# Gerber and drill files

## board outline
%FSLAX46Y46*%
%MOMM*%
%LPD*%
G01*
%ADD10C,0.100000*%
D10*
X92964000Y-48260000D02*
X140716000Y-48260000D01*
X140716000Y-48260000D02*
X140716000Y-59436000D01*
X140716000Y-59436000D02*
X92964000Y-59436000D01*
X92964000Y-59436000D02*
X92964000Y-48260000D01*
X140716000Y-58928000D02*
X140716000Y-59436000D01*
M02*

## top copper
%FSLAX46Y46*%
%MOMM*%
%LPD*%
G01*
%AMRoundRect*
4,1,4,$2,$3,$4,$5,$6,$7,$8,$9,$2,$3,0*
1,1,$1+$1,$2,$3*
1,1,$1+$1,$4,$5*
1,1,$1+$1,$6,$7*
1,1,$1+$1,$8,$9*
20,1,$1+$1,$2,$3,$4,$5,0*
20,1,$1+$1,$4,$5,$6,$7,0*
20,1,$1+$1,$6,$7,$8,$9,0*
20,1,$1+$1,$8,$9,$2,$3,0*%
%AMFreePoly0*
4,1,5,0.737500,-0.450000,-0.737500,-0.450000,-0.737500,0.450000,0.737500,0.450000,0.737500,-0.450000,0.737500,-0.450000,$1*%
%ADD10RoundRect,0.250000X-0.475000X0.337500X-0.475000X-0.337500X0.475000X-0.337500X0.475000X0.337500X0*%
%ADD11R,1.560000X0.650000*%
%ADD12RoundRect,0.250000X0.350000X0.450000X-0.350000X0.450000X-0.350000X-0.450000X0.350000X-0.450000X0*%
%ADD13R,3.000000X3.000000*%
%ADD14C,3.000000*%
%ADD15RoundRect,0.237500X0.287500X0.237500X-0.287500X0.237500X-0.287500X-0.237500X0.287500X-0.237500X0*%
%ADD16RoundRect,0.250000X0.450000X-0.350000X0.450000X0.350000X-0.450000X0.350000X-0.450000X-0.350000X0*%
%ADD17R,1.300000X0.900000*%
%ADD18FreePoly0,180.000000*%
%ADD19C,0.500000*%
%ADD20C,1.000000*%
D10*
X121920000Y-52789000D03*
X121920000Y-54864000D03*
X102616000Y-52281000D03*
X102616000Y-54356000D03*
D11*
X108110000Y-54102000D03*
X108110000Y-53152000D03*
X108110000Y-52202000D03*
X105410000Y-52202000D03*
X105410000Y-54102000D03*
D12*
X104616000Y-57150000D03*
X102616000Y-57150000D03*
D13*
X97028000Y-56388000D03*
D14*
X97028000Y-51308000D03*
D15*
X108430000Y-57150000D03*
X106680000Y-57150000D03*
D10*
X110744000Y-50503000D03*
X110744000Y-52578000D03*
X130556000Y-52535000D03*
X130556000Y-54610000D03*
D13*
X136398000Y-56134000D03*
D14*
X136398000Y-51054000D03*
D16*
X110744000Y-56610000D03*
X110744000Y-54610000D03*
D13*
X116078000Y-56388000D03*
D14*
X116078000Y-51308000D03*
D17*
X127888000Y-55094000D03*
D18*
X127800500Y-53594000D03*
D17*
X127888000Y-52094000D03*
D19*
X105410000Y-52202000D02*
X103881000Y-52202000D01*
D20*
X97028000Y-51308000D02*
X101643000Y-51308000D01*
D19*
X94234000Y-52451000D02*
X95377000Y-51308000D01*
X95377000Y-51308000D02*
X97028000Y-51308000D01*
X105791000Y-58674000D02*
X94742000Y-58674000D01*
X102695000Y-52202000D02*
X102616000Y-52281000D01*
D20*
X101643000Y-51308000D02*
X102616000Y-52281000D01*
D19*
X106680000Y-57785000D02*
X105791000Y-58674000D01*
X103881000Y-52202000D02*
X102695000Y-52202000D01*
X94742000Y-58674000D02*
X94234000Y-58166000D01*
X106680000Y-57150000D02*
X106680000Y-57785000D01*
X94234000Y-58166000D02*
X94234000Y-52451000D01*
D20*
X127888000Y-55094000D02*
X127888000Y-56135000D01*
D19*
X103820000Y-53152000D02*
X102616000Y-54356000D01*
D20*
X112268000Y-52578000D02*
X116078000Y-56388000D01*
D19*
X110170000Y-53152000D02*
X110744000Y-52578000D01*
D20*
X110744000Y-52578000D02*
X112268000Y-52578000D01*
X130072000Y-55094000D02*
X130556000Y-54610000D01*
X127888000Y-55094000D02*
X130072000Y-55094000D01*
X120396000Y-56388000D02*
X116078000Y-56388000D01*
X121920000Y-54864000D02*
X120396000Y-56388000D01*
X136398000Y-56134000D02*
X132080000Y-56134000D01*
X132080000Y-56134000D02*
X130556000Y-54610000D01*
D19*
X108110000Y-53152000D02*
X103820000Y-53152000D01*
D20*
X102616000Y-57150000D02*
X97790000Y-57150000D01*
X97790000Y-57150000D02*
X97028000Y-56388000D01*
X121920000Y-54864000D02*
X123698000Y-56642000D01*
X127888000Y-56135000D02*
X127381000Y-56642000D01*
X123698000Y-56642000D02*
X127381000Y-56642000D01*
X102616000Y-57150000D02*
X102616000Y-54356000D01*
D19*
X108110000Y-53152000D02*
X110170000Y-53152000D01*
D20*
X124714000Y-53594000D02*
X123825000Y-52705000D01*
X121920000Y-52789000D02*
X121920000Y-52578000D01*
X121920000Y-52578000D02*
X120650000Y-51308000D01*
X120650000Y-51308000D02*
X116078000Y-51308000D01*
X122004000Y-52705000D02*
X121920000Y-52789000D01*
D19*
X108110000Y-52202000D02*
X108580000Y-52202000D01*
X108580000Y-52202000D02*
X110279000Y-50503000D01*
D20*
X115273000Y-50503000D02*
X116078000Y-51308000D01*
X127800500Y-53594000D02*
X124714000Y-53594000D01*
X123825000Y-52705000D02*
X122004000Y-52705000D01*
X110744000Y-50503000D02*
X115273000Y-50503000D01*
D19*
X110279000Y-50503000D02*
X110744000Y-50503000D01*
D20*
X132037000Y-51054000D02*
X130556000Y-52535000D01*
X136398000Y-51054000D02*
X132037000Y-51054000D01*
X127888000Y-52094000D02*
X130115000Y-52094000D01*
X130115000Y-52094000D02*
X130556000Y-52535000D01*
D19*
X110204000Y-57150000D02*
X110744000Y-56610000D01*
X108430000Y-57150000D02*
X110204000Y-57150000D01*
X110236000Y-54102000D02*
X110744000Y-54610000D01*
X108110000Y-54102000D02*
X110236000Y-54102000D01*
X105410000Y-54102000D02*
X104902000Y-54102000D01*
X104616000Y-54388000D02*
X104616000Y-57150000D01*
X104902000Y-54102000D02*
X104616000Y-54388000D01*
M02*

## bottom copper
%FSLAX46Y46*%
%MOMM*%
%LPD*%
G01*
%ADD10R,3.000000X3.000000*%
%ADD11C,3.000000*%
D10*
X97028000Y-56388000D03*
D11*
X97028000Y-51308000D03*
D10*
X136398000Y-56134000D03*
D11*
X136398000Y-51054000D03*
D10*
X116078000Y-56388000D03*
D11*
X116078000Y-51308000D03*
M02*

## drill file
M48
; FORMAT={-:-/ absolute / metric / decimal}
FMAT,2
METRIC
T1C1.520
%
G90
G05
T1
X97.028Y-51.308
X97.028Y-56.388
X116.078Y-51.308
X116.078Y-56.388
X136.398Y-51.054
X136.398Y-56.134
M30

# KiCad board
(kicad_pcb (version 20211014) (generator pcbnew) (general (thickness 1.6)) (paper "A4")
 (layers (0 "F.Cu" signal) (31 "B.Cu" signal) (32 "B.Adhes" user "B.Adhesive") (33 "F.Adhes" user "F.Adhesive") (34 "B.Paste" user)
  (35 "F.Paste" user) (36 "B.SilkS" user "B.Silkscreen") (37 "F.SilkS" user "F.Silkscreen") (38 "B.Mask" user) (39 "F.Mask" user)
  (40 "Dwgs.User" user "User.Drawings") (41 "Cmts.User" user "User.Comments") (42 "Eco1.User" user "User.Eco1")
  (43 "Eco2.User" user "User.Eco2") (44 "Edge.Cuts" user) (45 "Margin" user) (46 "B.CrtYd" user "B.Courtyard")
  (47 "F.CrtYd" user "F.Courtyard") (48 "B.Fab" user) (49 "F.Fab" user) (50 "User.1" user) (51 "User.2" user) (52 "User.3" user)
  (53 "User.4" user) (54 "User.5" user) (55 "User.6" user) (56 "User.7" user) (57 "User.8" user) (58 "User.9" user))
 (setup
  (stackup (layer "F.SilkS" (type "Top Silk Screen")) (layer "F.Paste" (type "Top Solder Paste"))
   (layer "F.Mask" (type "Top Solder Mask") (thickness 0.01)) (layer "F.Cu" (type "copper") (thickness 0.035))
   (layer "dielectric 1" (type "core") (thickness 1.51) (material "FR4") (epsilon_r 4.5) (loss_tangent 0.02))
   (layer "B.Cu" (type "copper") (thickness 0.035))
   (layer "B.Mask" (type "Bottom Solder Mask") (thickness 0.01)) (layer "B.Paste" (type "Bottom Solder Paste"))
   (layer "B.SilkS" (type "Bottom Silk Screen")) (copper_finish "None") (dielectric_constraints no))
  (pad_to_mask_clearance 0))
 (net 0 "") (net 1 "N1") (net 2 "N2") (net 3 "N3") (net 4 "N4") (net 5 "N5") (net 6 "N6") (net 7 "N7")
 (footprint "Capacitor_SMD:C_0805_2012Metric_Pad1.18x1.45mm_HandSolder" (layer "F.Cu") (at 121.92 53.8265 -90)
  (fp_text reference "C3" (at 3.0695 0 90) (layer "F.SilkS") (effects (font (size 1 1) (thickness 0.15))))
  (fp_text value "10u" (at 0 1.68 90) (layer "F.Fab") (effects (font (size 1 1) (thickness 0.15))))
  (pad "1" smd roundrect (at -1.0375 0 270) (size 1.175 1.45) (layers "F.Cu" "F.Paste" "F.Mask") (roundrect_rratio 0.212766) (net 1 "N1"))
  (pad "2" smd roundrect (at 1.0375 0 270) (size 1.175 1.45) (layers "F.Cu" "F.Paste" "F.Mask") (roundrect_rratio 0.212766) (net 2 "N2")))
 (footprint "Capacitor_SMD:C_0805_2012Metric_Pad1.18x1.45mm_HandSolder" (layer "F.Cu") (at 102.616 53.3185 -90)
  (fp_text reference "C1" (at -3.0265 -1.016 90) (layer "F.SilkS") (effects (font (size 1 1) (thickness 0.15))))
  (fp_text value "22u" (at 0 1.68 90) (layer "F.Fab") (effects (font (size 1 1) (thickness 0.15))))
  (pad "1" smd roundrect (at -1.0375 0 270) (size 1.175 1.45) (layers "F.Cu" "F.Paste" "F.Mask") (roundrect_rratio 0.212766) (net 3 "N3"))
  (pad "2" smd roundrect (at 1.0375 0 270) (size 1.175 1.45) (layers "F.Cu" "F.Paste" "F.Mask") (roundrect_rratio 0.212766) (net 2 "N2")))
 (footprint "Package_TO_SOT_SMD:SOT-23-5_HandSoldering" (layer "F.Cu") (at 106.76 53.152 180)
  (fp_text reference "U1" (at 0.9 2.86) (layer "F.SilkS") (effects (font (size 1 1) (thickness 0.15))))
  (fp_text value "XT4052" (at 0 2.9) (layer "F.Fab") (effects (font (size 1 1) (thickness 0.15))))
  (pad "1" smd rect (at -1.35 -0.95 180) (size 1.56 0.65) (layers "F.Cu" "F.Paste" "F.Mask") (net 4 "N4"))
  (pad "2" smd rect (at -1.35 0 180) (size 1.56 0.65) (layers "F.Cu" "F.Paste" "F.Mask") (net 2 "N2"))
  (pad "3" smd rect (at -1.35 0.95 180) (size 1.56 0.65) (layers "F.Cu" "F.Paste" "F.Mask") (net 1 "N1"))
  (pad "4" smd rect (at 1.35 0.95 180) (size 1.56 0.65) (layers "F.Cu" "F.Paste" "F.Mask") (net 3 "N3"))
  (pad "5" smd rect (at 1.35 -0.95 180) (size 1.56 0.65) (layers "F.Cu" "F.Paste" "F.Mask") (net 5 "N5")))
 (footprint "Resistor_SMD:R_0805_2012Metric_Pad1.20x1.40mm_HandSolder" (layer "F.Cu") (at 103.616 57.15 180)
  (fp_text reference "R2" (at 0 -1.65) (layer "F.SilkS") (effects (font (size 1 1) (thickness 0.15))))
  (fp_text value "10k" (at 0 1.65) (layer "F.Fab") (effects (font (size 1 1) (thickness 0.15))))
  (pad "1" smd roundrect (at -1 0 180) (size 1.2 1.4) (layers "F.Cu" "F.Paste" "F.Mask") (roundrect_rratio 0.208333) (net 5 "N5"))
  (pad "2" smd roundrect (at 1 0 180) (size 1.2 1.4) (layers "F.Cu" "F.Paste" "F.Mask") (roundrect_rratio 0.208333) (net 2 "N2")))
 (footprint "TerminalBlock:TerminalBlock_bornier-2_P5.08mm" (layer "F.Cu") (at 97.028 56.388 90)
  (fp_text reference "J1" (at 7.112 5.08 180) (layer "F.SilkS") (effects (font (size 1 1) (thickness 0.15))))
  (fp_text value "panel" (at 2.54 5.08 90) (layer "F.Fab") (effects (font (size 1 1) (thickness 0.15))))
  (pad "1" thru_hole rect (at 0 0 90) (size 3 3) (drill 1.52) (layers *.Cu *.Mask) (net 2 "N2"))
  (pad "2" thru_hole circle (at 5.08 0 90) (size 3 3) (drill 1.52) (layers *.Cu *.Mask) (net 3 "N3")))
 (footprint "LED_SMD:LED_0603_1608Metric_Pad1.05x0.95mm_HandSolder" (layer "F.Cu") (at 107.555 57.15 180)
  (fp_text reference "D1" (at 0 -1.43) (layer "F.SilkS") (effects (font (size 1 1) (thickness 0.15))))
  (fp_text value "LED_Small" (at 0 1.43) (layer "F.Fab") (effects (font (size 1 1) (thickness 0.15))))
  (pad "1" smd roundrect (at -0.875 0 180) (size 1.05 0.95) (layers "F.Cu" "F.Paste" "F.Mask") (roundrect_rratio 0.25) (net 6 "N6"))
  (pad "2" smd roundrect (at 0.875 0 180) (size 1.05 0.95) (layers "F.Cu" "F.Paste" "F.Mask") (roundrect_rratio 0.25) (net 3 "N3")))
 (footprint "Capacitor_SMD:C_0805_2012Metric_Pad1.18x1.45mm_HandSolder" (layer "F.Cu") (at 110.744 51.5405 -90)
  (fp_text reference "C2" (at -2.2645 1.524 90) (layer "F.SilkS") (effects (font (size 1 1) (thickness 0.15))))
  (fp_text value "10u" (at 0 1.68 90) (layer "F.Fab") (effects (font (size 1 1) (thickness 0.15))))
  (pad "1" smd roundrect (at -1.0375 0 270) (size 1.175 1.45) (layers "F.Cu" "F.Paste" "F.Mask") (roundrect_rratio 0.212766) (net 1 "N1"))
  (pad "2" smd roundrect (at 1.0375 0 270) (size 1.175 1.45) (layers "F.Cu" "F.Paste" "F.Mask") (roundrect_rratio 0.212766) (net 2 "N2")))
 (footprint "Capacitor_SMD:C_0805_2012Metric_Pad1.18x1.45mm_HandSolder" (layer "F.Cu") (at 130.556 53.5725 -90)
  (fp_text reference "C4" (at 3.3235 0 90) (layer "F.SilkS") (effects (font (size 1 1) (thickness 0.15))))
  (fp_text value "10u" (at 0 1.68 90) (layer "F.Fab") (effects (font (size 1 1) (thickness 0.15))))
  (pad "1" smd roundrect (at -1.0375 0 270) (size 1.175 1.45) (layers "F.Cu" "F.Paste" "F.Mask") (roundrect_rratio 0.212766) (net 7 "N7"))
  (pad "2" smd roundrect (at 1.0375 0 270) (size 1.175 1.45) (layers "F.Cu" "F.Paste" "F.Mask") (roundrect_rratio 0.212766) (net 2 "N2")))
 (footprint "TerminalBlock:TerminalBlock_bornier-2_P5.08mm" (layer "F.Cu") (at 136.398 56.134 90)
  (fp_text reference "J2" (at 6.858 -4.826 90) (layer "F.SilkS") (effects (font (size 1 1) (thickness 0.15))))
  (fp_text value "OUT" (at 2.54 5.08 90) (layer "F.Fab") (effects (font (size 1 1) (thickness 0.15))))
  (pad "1" thru_hole rect (at 0 0 90) (size 3 3) (drill 1.52) (layers *.Cu *.Mask) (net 2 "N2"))
  (pad "2" thru_hole circle (at 5.08 0 90) (size 3 3) (drill 1.52) (layers *.Cu *.Mask) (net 7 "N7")))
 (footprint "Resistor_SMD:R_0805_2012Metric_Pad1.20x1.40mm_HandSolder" (layer "F.Cu") (at 110.744 55.61 90)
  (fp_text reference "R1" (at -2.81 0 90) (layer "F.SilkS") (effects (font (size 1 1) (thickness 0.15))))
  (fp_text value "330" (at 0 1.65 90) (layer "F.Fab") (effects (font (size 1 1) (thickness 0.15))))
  (pad "1" smd roundrect (at -1 0 90) (size 1.2 1.4) (layers "F.Cu" "F.Paste" "F.Mask") (roundrect_rratio 0.208333) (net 6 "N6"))
  (pad "2" smd roundrect (at 1 0 90) (size 1.2 1.4) (layers "F.Cu" "F.Paste" "F.Mask") (roundrect_rratio 0.208333) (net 4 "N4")))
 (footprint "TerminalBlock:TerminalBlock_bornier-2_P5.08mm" (layer "F.Cu") (at 116.078 56.388 90)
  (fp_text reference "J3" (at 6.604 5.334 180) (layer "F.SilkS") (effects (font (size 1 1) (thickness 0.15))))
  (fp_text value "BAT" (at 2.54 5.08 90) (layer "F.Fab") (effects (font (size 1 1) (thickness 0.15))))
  (pad "1" thru_hole rect (at 0 0 90) (size 3 3) (drill 1.52) (layers *.Cu *.Mask) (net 2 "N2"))
  (pad "2" thru_hole circle (at 5.08 0 90) (size 3 3) (drill 1.52) (layers *.Cu *.Mask) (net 1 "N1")))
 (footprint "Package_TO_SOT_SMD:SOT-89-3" (layer "F.Cu") (at 126.238 53.594 180)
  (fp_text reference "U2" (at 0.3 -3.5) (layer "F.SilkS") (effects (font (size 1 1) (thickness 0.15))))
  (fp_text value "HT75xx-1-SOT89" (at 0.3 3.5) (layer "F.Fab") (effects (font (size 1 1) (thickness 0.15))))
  (pad "1" smd rect (at -1.65 -1.5 180) (size 1.3 0.9) (layers "F.Cu" "F.Paste" "F.Mask") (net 2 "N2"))
  (pad "2" smd custom (at -1.5625 0 180) (size 1.475 0.9) (layers "F.Cu" "F.Paste" "F.Mask") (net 1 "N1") (zone_connect 2)
   (options (clearance outline) (anchor rect)) (primitives))
  (pad "3" smd rect (at -1.65 1.5 180) (size 1.3 0.9) (layers "F.Cu" "F.Paste" "F.Mask") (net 7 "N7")))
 (gr_line (start 92.964 48.26) (end 140.716 48.26) (layer "Edge.Cuts") (width 0.1))
 (gr_line (start 140.716 48.26) (end 140.716 59.436) (layer "Edge.Cuts") (width 0.1))
 (gr_line (start 140.716 59.436) (end 92.964 59.436) (layer "Edge.Cuts") (width 0.1))
 (gr_line (start 92.964 59.436) (end 92.964 48.26) (layer "Edge.Cuts") (width 0.1))
 (gr_line (start 140.716 58.928) (end 140.716 59.436) (layer "Edge.Cuts") (width 0.1))
 (segment (start 105.41 52.202) (end 103.881 52.202) (width 0.5) (layer "F.Cu") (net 3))
 (segment (start 97.028 51.308) (end 101.643 51.308) (width 1) (layer "F.Cu") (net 3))
 (segment (start 94.234 52.451) (end 95.377 51.308) (width 0.5) (layer "F.Cu") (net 3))
 (segment (start 95.377 51.308) (end 97.028 51.308) (width 0.5) (layer "F.Cu") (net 3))
 (segment (start 105.791 58.674) (end 94.742 58.674) (width 0.5) (layer "F.Cu") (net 3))
 (segment (start 102.695 52.202) (end 102.616 52.281) (width 0.5) (layer "F.Cu") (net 3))
 (segment (start 101.643 51.308) (end 102.616 52.281) (width 1) (layer "F.Cu") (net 3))
 (segment (start 106.68 57.785) (end 105.791 58.674) (width 0.5) (layer "F.Cu") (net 3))
 (segment (start 103.881 52.202) (end 102.695 52.202) (width 0.5) (layer "F.Cu") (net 3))
 (segment (start 94.742 58.674) (end 94.234 58.166) (width 0.5) (layer "F.Cu") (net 3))
 (segment (start 106.68 57.15) (end 106.68 57.785) (width 0.5) (layer "F.Cu") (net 3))
 (segment (start 94.234 58.166) (end 94.234 52.451) (width 0.5) (layer "F.Cu") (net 3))
 (segment (start 127.888 55.094) (end 127.888 56.135) (width 1) (layer "F.Cu") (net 2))
 (segment (start 103.82 53.152) (end 102.616 54.356) (width 0.5) (layer "F.Cu") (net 2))
 (segment (start 112.268 52.578) (end 116.078 56.388) (width 1) (layer "F.Cu") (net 2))
 (segment (start 110.17 53.152) (end 110.744 52.578) (width 0.5) (layer "F.Cu") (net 2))
 (segment (start 110.744 52.578) (end 112.268 52.578) (width 1) (layer "F.Cu") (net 2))
 (segment (start 130.072 55.094) (end 130.556 54.61) (width 1) (layer "F.Cu") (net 2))
 (segment (start 127.888 55.094) (end 130.072 55.094) (width 1) (layer "F.Cu") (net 2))
 (segment (start 120.396 56.388) (end 116.078 56.388) (width 1) (layer "F.Cu") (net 2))
 (segment (start 121.92 54.864) (end 120.396 56.388) (width 1) (layer "F.Cu") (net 2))
 (segment (start 136.398 56.134) (end 132.08 56.134) (width 1) (layer "F.Cu") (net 2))
 (segment (start 132.08 56.134) (end 130.556 54.61) (width 1) (layer "F.Cu") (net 2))
 (segment (start 108.11 53.152) (end 103.82 53.152) (width 0.5) (layer "F.Cu") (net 2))
 (segment (start 102.616 57.15) (end 97.79 57.15) (width 1) (layer "F.Cu") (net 2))
 (segment (start 97.79 57.15) (end 97.028 56.388) (width 1) (layer "F.Cu") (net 2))
 (segment (start 121.92 54.864) (end 123.698 56.642) (width 1) (layer "F.Cu") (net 2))
 (segment (start 127.888 56.135) (end 127.381 56.642) (width 1) (layer "F.Cu") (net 2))
 (segment (start 123.698 56.642) (end 127.381 56.642) (width 1) (layer "F.Cu") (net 2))
 (segment (start 102.616 57.15) (end 102.616 54.356) (width 1) (layer "F.Cu") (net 2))
 (segment (start 108.11 53.152) (end 110.17 53.152) (width 0.5) (layer "F.Cu") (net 2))
 (segment (start 124.714 53.594) (end 123.825 52.705) (width 1) (layer "F.Cu") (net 1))
 (segment (start 121.92 52.789) (end 121.92 52.578) (width 1) (layer "F.Cu") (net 1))
 (segment (start 121.92 52.578) (end 120.65 51.308) (width 1) (layer "F.Cu") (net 1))
 (segment (start 120.65 51.308) (end 116.078 51.308) (width 1) (layer "F.Cu") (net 1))
 (segment (start 122.004 52.705) (end 121.92 52.789) (width 1) (layer "F.Cu") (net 1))
 (segment (start 108.11 52.202) (end 108.58 52.202) (width 0.5) (layer "F.Cu") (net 1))
 (segment (start 108.58 52.202) (end 110.279 50.503) (width 0.5) (layer "F.Cu") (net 1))
 (segment (start 115.273 50.503) (end 116.078 51.308) (width 1) (layer "F.Cu") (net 1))
 (segment (start 127.8005 53.594) (end 124.714 53.594) (width 1) (layer "F.Cu") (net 1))
 (segment (start 123.825 52.705) (end 122.004 52.705) (width 1) (layer "F.Cu") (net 1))
 (segment (start 110.744 50.503) (end 115.273 50.503) (width 1) (layer "F.Cu") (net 1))
 (segment (start 110.279 50.503) (end 110.744 50.503) (width 0.5) (layer "F.Cu") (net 1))
 (segment (start 132.037 51.054) (end 130.556 52.535) (width 1) (layer "F.Cu") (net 7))
 (segment (start 136.398 51.054) (end 132.037 51.054) (width 1) (layer "F.Cu") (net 7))
 (segment (start 127.888 52.094) (end 130.115 52.094) (width 1) (layer "F.Cu") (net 7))
 (segment (start 130.115 52.094) (end 130.556 52.535) (width 1) (layer "F.Cu") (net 7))
 (segment (start 110.204 57.15) (end 110.744 56.61) (width 0.5) (layer "F.Cu") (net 6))
 (segment (start 108.43 57.15) (end 110.204 57.15) (width 0.5) (layer "F.Cu") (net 6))
 (segment (start 110.236 54.102) (end 110.744 54.61) (width 0.5) (layer "F.Cu") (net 4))
 (segment (start 108.11 54.102) (end 110.236 54.102) (width 0.5) (layer "F.Cu") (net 4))
 (segment (start 105.41 54.102) (end 104.902 54.102) (width 0.5) (layer "F.Cu") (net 5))
 (segment (start 104.616 54.388) (end 104.616 57.15) (width 0.5) (layer "F.Cu") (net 5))
 (segment (start 104.902 54.102) (end 104.616 54.388) (width 0.5) (layer "F.Cu") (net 5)))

